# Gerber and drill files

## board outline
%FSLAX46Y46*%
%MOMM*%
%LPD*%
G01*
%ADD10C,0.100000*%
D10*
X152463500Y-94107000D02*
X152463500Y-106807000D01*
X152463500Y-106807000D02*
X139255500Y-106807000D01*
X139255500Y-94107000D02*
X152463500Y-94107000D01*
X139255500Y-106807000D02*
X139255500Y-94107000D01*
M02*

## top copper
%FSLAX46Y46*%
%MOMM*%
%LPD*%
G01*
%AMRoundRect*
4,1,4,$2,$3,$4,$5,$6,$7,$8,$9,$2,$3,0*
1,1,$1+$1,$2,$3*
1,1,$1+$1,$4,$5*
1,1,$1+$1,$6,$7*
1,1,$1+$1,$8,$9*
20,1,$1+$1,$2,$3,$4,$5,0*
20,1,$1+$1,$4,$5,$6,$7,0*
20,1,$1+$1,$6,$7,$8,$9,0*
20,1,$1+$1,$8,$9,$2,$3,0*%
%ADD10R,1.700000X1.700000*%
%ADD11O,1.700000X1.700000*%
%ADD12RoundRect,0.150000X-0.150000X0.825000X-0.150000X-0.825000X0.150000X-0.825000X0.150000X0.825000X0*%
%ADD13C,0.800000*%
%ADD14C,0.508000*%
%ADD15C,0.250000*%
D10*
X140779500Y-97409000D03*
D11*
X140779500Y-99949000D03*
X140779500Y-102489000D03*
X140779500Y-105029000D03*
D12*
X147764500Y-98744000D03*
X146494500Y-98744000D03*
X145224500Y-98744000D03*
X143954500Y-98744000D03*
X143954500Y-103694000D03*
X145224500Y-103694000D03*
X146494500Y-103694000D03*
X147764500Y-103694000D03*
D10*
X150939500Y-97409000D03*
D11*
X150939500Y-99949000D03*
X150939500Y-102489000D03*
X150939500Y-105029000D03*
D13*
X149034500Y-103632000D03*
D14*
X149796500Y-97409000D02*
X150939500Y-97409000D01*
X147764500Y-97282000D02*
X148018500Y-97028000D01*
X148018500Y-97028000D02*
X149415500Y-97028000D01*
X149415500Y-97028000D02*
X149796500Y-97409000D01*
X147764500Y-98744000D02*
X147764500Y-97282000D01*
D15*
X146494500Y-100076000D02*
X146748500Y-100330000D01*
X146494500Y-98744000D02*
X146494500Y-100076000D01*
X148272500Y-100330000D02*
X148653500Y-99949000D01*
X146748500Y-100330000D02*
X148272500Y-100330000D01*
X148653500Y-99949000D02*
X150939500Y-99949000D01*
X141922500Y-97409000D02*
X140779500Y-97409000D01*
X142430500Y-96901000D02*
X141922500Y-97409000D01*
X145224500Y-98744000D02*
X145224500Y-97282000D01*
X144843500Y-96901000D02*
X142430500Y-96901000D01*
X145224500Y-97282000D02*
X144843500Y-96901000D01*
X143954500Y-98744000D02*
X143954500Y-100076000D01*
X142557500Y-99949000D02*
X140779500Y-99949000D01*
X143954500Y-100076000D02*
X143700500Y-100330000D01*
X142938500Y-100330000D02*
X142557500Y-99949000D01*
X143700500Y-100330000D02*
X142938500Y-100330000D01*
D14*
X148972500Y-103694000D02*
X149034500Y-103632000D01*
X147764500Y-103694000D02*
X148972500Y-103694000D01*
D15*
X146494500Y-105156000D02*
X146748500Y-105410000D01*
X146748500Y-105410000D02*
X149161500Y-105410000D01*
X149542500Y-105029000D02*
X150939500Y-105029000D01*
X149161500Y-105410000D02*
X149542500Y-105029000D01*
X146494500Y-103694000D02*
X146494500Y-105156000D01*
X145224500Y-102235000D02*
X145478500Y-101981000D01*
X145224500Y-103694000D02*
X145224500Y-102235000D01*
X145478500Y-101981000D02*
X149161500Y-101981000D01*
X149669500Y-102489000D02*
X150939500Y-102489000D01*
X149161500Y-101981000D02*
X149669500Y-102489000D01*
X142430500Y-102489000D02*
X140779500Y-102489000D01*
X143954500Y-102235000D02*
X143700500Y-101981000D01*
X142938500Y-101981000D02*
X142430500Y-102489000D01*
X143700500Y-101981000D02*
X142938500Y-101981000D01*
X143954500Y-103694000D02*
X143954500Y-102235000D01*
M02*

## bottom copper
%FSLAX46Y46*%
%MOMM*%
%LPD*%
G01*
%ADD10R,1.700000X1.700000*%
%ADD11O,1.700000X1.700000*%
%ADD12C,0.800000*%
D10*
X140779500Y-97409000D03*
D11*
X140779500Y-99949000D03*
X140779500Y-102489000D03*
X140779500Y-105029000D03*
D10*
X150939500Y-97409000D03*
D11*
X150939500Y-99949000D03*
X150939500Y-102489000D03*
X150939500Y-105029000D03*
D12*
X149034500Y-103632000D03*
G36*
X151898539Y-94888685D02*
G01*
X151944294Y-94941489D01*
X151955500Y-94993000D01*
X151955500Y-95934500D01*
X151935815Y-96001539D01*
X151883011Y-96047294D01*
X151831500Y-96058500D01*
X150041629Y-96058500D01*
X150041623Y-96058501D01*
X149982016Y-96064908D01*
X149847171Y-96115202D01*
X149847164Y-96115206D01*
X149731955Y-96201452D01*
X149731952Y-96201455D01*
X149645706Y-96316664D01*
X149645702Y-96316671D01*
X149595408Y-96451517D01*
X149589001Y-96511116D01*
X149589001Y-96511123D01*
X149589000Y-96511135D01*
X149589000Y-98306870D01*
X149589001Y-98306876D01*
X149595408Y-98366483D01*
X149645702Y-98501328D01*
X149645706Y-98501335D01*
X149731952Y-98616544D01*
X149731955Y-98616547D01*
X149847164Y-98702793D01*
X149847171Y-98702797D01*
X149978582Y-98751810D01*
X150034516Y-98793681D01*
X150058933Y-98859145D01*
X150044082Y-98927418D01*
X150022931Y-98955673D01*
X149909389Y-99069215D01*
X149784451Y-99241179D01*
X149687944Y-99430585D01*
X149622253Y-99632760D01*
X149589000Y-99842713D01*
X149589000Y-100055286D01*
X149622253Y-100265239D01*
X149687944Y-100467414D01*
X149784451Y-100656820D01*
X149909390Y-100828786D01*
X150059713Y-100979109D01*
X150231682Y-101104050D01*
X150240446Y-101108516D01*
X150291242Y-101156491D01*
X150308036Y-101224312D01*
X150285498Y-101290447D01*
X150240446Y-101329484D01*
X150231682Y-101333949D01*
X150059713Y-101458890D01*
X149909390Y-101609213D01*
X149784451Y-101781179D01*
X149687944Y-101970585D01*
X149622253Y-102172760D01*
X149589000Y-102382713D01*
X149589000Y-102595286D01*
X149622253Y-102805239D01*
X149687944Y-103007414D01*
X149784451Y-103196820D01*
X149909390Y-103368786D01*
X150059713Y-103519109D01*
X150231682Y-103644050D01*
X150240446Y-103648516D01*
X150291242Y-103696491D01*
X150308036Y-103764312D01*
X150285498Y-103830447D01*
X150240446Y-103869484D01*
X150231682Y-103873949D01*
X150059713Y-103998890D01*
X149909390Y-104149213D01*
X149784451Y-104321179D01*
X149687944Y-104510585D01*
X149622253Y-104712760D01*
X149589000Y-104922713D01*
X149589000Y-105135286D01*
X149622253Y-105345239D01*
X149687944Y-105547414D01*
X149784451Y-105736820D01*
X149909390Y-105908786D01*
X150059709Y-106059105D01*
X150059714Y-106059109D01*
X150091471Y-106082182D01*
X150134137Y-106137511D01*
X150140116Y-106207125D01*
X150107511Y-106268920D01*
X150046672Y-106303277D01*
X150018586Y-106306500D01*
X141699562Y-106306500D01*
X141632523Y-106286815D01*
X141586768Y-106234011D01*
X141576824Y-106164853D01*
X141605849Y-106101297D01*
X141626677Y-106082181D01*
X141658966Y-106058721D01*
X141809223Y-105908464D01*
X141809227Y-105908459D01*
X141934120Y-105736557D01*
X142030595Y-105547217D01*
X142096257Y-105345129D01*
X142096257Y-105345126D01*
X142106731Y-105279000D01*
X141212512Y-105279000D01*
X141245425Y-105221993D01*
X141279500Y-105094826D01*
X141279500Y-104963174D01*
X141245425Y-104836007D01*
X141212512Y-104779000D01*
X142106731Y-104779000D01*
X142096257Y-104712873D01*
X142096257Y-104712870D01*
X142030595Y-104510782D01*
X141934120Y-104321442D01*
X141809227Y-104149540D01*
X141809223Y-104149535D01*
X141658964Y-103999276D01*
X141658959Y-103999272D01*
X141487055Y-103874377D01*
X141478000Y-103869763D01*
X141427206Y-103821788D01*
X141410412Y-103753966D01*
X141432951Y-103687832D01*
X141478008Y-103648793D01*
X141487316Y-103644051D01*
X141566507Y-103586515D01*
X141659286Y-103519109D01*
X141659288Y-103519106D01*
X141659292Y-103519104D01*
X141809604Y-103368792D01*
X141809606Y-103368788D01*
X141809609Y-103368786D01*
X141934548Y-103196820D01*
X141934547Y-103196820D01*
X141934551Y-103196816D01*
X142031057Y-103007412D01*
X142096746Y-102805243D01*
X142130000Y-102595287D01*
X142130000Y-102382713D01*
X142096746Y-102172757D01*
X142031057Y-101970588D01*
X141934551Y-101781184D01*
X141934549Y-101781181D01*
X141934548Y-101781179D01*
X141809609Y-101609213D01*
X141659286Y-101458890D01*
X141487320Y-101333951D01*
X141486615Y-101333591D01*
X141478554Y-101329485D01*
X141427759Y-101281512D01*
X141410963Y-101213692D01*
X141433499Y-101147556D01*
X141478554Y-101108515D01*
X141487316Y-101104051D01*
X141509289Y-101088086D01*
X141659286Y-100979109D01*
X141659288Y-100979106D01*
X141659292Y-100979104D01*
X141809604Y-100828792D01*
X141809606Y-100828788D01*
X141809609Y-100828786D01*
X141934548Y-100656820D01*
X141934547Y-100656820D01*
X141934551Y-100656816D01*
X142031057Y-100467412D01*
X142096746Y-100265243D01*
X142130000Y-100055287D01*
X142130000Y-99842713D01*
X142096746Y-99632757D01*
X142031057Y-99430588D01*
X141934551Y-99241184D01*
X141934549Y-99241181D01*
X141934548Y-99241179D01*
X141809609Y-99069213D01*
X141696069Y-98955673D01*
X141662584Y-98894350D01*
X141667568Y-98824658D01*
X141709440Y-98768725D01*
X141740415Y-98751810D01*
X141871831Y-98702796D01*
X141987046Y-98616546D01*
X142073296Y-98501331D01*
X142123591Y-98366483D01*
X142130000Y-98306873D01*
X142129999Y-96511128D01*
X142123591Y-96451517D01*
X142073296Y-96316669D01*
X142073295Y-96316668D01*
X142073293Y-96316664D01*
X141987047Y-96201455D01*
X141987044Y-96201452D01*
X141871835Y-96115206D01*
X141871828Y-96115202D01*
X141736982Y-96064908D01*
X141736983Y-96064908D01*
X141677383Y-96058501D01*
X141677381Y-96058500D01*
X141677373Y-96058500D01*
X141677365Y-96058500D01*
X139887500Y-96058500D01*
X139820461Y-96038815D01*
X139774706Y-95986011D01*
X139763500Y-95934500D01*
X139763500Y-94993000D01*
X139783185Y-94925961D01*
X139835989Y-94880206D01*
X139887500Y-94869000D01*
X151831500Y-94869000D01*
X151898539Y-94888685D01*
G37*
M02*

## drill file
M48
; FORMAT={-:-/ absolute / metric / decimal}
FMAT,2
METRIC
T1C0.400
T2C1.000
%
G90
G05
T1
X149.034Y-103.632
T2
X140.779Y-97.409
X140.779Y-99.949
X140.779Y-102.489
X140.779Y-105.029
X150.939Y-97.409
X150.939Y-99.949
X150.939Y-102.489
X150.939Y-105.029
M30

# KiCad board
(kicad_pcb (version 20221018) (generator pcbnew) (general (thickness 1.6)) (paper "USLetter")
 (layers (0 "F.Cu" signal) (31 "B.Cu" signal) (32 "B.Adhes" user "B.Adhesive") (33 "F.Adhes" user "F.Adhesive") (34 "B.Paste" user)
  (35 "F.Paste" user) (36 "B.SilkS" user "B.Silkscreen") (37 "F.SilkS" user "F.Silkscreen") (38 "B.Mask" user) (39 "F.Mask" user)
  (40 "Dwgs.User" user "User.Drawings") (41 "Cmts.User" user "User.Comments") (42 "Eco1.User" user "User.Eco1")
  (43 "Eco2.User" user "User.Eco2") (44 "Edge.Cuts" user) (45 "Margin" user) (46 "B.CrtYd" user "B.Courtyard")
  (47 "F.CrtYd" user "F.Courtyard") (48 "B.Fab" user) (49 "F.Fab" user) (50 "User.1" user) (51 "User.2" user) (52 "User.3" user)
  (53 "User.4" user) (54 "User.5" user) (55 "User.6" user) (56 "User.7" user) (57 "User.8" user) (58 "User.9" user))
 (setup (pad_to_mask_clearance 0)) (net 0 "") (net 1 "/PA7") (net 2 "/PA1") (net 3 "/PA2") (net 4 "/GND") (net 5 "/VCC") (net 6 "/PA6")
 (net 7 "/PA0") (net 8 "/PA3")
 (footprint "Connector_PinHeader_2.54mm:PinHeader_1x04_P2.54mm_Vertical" (layer "F.Cu") (at 140.7795 97.409)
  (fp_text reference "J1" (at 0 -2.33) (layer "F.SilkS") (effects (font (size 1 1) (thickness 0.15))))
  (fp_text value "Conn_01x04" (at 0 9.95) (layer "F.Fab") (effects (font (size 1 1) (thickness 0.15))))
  (pad "1" thru_hole rect (at 0 0) (size 1.7 1.7) (drill 1) (layers "*.Cu" "*.Mask") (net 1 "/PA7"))
  (pad "2" thru_hole oval (at 0 2.54) (size 1.7 1.7) (drill 1) (layers "*.Cu" "*.Mask") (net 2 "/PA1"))
  (pad "3" thru_hole oval (at 0 5.08) (size 1.7 1.7) (drill 1) (layers "*.Cu" "*.Mask") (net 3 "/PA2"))
  (pad "4" thru_hole oval (at 0 7.62) (size 1.7 1.7) (drill 1) (layers "*.Cu" "*.Mask") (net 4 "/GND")))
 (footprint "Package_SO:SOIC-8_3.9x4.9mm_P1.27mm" (layer "F.Cu") (at 145.8595 101.219 -90)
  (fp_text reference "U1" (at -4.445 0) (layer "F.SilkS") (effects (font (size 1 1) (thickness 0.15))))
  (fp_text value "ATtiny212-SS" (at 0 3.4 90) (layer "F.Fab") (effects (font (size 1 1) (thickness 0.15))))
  (pad "1" smd roundrect (at -2.475 -1.905 270) (size 1.95 0.6) (layers "F.Cu" "F.Paste" "F.Mask") (roundrect_rratio 0.25) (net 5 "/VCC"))
  (pad "2" smd roundrect (at -2.475 -0.635 270) (size 1.95 0.6) (layers "F.Cu" "F.Paste" "F.Mask") (roundrect_rratio 0.25) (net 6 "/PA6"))
  (pad "3" smd roundrect (at -2.475 0.635 270) (size 1.95 0.6) (layers "F.Cu" "F.Paste" "F.Mask") (roundrect_rratio 0.25) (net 1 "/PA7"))
  (pad "4" smd roundrect (at -2.475 1.905 270) (size 1.95 0.6) (layers "F.Cu" "F.Paste" "F.Mask") (roundrect_rratio 0.25) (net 2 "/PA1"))
  (pad "5" smd roundrect (at 2.475 1.905 270) (size 1.95 0.6) (layers "F.Cu" "F.Paste" "F.Mask") (roundrect_rratio 0.25) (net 3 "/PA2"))
  (pad "6" smd roundrect (at 2.475 0.635 270) (size 1.95 0.6) (layers "F.Cu" "F.Paste" "F.Mask") (roundrect_rratio 0.25) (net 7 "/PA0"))
  (pad "7" smd roundrect (at 2.475 -0.635 270) (size 1.95 0.6) (layers "F.Cu" "F.Paste" "F.Mask") (roundrect_rratio 0.25) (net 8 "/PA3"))
  (pad "8" smd roundrect (at 2.475 -1.905 270) (size 1.95 0.6) (layers "F.Cu" "F.Paste" "F.Mask") (roundrect_rratio 0.25) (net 4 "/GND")))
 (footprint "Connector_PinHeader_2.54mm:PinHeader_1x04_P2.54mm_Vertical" (layer "F.Cu") (at 150.9395 97.409)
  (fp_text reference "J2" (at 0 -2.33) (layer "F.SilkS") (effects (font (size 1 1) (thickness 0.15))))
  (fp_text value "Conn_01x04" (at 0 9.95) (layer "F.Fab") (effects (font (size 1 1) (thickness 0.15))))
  (pad "1" thru_hole rect (at 0 0) (size 1.7 1.7) (drill 1) (layers "*.Cu" "*.Mask") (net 5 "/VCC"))
  (pad "2" thru_hole oval (at 0 2.54) (size 1.7 1.7) (drill 1) (layers "*.Cu" "*.Mask") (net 6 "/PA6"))
  (pad "3" thru_hole oval (at 0 5.08) (size 1.7 1.7) (drill 1) (layers "*.Cu" "*.Mask") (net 7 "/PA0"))
  (pad "4" thru_hole oval (at 0 7.62) (size 1.7 1.7) (drill 1) (layers "*.Cu" "*.Mask") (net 8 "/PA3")))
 (gr_line (start 152.4635 94.107) (end 152.4635 106.807) (stroke (width 0.1) (type default)) (layer "Edge.Cuts"))
 (gr_line (start 152.4635 106.807) (end 139.2555 106.807) (stroke (width 0.1) (type default)) (layer "Edge.Cuts"))
 (gr_line (start 139.2555 94.107) (end 152.4635 94.107) (stroke (width 0.1) (type default)) (layer "Edge.Cuts"))
 (gr_line (start 139.2555 106.807) (end 139.2555 94.107) (stroke (width 0.1) (type default)) (layer "Edge.Cuts"))
 (segment (start 149.7965 97.409) (end 150.9395 97.409) (width 0.508) (layer "F.Cu") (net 5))
 (segment (start 147.7645 97.282) (end 148.0185 97.028) (width 0.508) (layer "F.Cu") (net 5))
 (segment (start 148.0185 97.028) (end 149.4155 97.028) (width 0.508) (layer "F.Cu") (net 5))
 (segment (start 149.4155 97.028) (end 149.7965 97.409) (width 0.508) (layer "F.Cu") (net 5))
 (segment (start 147.7645 98.744) (end 147.7645 97.282) (width 0.508) (layer "F.Cu") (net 5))
 (segment (start 146.4945 100.076) (end 146.7485 100.33) (width 0.25) (layer "F.Cu") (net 6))
 (segment (start 146.4945 98.744) (end 146.4945 100.076) (width 0.25) (layer "F.Cu") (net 6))
 (segment (start 148.2725 100.33) (end 148.6535 99.949) (width 0.25) (layer "F.Cu") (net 6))
 (segment (start 146.7485 100.33) (end 148.2725 100.33) (width 0.25) (layer "F.Cu") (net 6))
 (segment (start 148.6535 99.949) (end 150.9395 99.949) (width 0.25) (layer "F.Cu") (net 6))
 (segment (start 141.9225 97.409) (end 140.7795 97.409) (width 0.25) (layer "F.Cu") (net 1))
 (segment (start 142.4305 96.901) (end 141.9225 97.409) (width 0.25) (layer "F.Cu") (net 1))
 (segment (start 145.2245 98.744) (end 145.2245 97.282) (width 0.25) (layer "F.Cu") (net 1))
 (segment (start 144.8435 96.901) (end 142.4305 96.901) (width 0.25) (layer "F.Cu") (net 1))
 (segment (start 145.2245 97.282) (end 144.8435 96.901) (width 0.25) (layer "F.Cu") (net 1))
 (segment (start 143.9545 98.744) (end 143.9545 100.076) (width 0.25) (layer "F.Cu") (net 2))
 (segment (start 142.5575 99.949) (end 140.7795 99.949) (width 0.25) (layer "F.Cu") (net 2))
 (segment (start 143.9545 100.076) (end 143.7005 100.33) (width 0.25) (layer "F.Cu") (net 2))
 (segment (start 142.9385 100.33) (end 142.5575 99.949) (width 0.25) (layer "F.Cu") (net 2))
 (segment (start 143.7005 100.33) (end 142.9385 100.33) (width 0.25) (layer "F.Cu") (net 2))
 (segment (start 148.9725 103.694) (end 149.0345 103.632) (width 0.508) (layer "F.Cu") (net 4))
 (segment (start 147.7645 103.694) (end 148.9725 103.694) (width 0.508) (layer "F.Cu") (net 4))
 (via (at 149.0345 103.632) (size 0.8) (drill 0.4) (layers "F.Cu" "B.Cu") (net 4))
 (segment (start 146.4945 105.156) (end 146.7485 105.41) (width 0.25) (layer "F.Cu") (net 8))
 (segment (start 146.7485 105.41) (end 149.1615 105.41) (width 0.25) (layer "F.Cu") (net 8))
 (segment (start 149.5425 105.029) (end 150.9395 105.029) (width 0.25) (layer "F.Cu") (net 8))
 (segment (start 149.1615 105.41) (end 149.5425 105.029) (width 0.25) (layer "F.Cu") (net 8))
 (segment (start 146.4945 103.694) (end 146.4945 105.156) (width 0.25) (layer "F.Cu") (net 8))
 (segment (start 145.2245 102.235) (end 145.4785 101.981) (width 0.25) (layer "F.Cu") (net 7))
 (segment (start 145.2245 103.694) (end 145.2245 102.235) (width 0.25) (layer "F.Cu") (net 7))
 (segment (start 145.4785 101.981) (end 149.1615 101.981) (width 0.25) (layer "F.Cu") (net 7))
 (segment (start 149.6695 102.489) (end 150.9395 102.489) (width 0.25) (layer "F.Cu") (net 7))
 (segment (start 149.1615 101.981) (end 149.6695 102.489) (width 0.25) (layer "F.Cu") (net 7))
 (segment (start 142.4305 102.489) (end 140.7795 102.489) (width 0.25) (layer "F.Cu") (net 3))
 (segment (start 143.9545 102.235) (end 143.7005 101.981) (width 0.25) (layer "F.Cu") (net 3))
 (segment (start 142.9385 101.981) (end 142.4305 102.489) (width 0.25) (layer "F.Cu") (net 3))
 (segment (start 143.7005 101.981) (end 142.9385 101.981) (width 0.25) (layer "F.Cu") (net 3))
 (segment (start 143.9545 103.694) (end 143.9545 102.235) (width 0.25) (layer "F.Cu") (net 3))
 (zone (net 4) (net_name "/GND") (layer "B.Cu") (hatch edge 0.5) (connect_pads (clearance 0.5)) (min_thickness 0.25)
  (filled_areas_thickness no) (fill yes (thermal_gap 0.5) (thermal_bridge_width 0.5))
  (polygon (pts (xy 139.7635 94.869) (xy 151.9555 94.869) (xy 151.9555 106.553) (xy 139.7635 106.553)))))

